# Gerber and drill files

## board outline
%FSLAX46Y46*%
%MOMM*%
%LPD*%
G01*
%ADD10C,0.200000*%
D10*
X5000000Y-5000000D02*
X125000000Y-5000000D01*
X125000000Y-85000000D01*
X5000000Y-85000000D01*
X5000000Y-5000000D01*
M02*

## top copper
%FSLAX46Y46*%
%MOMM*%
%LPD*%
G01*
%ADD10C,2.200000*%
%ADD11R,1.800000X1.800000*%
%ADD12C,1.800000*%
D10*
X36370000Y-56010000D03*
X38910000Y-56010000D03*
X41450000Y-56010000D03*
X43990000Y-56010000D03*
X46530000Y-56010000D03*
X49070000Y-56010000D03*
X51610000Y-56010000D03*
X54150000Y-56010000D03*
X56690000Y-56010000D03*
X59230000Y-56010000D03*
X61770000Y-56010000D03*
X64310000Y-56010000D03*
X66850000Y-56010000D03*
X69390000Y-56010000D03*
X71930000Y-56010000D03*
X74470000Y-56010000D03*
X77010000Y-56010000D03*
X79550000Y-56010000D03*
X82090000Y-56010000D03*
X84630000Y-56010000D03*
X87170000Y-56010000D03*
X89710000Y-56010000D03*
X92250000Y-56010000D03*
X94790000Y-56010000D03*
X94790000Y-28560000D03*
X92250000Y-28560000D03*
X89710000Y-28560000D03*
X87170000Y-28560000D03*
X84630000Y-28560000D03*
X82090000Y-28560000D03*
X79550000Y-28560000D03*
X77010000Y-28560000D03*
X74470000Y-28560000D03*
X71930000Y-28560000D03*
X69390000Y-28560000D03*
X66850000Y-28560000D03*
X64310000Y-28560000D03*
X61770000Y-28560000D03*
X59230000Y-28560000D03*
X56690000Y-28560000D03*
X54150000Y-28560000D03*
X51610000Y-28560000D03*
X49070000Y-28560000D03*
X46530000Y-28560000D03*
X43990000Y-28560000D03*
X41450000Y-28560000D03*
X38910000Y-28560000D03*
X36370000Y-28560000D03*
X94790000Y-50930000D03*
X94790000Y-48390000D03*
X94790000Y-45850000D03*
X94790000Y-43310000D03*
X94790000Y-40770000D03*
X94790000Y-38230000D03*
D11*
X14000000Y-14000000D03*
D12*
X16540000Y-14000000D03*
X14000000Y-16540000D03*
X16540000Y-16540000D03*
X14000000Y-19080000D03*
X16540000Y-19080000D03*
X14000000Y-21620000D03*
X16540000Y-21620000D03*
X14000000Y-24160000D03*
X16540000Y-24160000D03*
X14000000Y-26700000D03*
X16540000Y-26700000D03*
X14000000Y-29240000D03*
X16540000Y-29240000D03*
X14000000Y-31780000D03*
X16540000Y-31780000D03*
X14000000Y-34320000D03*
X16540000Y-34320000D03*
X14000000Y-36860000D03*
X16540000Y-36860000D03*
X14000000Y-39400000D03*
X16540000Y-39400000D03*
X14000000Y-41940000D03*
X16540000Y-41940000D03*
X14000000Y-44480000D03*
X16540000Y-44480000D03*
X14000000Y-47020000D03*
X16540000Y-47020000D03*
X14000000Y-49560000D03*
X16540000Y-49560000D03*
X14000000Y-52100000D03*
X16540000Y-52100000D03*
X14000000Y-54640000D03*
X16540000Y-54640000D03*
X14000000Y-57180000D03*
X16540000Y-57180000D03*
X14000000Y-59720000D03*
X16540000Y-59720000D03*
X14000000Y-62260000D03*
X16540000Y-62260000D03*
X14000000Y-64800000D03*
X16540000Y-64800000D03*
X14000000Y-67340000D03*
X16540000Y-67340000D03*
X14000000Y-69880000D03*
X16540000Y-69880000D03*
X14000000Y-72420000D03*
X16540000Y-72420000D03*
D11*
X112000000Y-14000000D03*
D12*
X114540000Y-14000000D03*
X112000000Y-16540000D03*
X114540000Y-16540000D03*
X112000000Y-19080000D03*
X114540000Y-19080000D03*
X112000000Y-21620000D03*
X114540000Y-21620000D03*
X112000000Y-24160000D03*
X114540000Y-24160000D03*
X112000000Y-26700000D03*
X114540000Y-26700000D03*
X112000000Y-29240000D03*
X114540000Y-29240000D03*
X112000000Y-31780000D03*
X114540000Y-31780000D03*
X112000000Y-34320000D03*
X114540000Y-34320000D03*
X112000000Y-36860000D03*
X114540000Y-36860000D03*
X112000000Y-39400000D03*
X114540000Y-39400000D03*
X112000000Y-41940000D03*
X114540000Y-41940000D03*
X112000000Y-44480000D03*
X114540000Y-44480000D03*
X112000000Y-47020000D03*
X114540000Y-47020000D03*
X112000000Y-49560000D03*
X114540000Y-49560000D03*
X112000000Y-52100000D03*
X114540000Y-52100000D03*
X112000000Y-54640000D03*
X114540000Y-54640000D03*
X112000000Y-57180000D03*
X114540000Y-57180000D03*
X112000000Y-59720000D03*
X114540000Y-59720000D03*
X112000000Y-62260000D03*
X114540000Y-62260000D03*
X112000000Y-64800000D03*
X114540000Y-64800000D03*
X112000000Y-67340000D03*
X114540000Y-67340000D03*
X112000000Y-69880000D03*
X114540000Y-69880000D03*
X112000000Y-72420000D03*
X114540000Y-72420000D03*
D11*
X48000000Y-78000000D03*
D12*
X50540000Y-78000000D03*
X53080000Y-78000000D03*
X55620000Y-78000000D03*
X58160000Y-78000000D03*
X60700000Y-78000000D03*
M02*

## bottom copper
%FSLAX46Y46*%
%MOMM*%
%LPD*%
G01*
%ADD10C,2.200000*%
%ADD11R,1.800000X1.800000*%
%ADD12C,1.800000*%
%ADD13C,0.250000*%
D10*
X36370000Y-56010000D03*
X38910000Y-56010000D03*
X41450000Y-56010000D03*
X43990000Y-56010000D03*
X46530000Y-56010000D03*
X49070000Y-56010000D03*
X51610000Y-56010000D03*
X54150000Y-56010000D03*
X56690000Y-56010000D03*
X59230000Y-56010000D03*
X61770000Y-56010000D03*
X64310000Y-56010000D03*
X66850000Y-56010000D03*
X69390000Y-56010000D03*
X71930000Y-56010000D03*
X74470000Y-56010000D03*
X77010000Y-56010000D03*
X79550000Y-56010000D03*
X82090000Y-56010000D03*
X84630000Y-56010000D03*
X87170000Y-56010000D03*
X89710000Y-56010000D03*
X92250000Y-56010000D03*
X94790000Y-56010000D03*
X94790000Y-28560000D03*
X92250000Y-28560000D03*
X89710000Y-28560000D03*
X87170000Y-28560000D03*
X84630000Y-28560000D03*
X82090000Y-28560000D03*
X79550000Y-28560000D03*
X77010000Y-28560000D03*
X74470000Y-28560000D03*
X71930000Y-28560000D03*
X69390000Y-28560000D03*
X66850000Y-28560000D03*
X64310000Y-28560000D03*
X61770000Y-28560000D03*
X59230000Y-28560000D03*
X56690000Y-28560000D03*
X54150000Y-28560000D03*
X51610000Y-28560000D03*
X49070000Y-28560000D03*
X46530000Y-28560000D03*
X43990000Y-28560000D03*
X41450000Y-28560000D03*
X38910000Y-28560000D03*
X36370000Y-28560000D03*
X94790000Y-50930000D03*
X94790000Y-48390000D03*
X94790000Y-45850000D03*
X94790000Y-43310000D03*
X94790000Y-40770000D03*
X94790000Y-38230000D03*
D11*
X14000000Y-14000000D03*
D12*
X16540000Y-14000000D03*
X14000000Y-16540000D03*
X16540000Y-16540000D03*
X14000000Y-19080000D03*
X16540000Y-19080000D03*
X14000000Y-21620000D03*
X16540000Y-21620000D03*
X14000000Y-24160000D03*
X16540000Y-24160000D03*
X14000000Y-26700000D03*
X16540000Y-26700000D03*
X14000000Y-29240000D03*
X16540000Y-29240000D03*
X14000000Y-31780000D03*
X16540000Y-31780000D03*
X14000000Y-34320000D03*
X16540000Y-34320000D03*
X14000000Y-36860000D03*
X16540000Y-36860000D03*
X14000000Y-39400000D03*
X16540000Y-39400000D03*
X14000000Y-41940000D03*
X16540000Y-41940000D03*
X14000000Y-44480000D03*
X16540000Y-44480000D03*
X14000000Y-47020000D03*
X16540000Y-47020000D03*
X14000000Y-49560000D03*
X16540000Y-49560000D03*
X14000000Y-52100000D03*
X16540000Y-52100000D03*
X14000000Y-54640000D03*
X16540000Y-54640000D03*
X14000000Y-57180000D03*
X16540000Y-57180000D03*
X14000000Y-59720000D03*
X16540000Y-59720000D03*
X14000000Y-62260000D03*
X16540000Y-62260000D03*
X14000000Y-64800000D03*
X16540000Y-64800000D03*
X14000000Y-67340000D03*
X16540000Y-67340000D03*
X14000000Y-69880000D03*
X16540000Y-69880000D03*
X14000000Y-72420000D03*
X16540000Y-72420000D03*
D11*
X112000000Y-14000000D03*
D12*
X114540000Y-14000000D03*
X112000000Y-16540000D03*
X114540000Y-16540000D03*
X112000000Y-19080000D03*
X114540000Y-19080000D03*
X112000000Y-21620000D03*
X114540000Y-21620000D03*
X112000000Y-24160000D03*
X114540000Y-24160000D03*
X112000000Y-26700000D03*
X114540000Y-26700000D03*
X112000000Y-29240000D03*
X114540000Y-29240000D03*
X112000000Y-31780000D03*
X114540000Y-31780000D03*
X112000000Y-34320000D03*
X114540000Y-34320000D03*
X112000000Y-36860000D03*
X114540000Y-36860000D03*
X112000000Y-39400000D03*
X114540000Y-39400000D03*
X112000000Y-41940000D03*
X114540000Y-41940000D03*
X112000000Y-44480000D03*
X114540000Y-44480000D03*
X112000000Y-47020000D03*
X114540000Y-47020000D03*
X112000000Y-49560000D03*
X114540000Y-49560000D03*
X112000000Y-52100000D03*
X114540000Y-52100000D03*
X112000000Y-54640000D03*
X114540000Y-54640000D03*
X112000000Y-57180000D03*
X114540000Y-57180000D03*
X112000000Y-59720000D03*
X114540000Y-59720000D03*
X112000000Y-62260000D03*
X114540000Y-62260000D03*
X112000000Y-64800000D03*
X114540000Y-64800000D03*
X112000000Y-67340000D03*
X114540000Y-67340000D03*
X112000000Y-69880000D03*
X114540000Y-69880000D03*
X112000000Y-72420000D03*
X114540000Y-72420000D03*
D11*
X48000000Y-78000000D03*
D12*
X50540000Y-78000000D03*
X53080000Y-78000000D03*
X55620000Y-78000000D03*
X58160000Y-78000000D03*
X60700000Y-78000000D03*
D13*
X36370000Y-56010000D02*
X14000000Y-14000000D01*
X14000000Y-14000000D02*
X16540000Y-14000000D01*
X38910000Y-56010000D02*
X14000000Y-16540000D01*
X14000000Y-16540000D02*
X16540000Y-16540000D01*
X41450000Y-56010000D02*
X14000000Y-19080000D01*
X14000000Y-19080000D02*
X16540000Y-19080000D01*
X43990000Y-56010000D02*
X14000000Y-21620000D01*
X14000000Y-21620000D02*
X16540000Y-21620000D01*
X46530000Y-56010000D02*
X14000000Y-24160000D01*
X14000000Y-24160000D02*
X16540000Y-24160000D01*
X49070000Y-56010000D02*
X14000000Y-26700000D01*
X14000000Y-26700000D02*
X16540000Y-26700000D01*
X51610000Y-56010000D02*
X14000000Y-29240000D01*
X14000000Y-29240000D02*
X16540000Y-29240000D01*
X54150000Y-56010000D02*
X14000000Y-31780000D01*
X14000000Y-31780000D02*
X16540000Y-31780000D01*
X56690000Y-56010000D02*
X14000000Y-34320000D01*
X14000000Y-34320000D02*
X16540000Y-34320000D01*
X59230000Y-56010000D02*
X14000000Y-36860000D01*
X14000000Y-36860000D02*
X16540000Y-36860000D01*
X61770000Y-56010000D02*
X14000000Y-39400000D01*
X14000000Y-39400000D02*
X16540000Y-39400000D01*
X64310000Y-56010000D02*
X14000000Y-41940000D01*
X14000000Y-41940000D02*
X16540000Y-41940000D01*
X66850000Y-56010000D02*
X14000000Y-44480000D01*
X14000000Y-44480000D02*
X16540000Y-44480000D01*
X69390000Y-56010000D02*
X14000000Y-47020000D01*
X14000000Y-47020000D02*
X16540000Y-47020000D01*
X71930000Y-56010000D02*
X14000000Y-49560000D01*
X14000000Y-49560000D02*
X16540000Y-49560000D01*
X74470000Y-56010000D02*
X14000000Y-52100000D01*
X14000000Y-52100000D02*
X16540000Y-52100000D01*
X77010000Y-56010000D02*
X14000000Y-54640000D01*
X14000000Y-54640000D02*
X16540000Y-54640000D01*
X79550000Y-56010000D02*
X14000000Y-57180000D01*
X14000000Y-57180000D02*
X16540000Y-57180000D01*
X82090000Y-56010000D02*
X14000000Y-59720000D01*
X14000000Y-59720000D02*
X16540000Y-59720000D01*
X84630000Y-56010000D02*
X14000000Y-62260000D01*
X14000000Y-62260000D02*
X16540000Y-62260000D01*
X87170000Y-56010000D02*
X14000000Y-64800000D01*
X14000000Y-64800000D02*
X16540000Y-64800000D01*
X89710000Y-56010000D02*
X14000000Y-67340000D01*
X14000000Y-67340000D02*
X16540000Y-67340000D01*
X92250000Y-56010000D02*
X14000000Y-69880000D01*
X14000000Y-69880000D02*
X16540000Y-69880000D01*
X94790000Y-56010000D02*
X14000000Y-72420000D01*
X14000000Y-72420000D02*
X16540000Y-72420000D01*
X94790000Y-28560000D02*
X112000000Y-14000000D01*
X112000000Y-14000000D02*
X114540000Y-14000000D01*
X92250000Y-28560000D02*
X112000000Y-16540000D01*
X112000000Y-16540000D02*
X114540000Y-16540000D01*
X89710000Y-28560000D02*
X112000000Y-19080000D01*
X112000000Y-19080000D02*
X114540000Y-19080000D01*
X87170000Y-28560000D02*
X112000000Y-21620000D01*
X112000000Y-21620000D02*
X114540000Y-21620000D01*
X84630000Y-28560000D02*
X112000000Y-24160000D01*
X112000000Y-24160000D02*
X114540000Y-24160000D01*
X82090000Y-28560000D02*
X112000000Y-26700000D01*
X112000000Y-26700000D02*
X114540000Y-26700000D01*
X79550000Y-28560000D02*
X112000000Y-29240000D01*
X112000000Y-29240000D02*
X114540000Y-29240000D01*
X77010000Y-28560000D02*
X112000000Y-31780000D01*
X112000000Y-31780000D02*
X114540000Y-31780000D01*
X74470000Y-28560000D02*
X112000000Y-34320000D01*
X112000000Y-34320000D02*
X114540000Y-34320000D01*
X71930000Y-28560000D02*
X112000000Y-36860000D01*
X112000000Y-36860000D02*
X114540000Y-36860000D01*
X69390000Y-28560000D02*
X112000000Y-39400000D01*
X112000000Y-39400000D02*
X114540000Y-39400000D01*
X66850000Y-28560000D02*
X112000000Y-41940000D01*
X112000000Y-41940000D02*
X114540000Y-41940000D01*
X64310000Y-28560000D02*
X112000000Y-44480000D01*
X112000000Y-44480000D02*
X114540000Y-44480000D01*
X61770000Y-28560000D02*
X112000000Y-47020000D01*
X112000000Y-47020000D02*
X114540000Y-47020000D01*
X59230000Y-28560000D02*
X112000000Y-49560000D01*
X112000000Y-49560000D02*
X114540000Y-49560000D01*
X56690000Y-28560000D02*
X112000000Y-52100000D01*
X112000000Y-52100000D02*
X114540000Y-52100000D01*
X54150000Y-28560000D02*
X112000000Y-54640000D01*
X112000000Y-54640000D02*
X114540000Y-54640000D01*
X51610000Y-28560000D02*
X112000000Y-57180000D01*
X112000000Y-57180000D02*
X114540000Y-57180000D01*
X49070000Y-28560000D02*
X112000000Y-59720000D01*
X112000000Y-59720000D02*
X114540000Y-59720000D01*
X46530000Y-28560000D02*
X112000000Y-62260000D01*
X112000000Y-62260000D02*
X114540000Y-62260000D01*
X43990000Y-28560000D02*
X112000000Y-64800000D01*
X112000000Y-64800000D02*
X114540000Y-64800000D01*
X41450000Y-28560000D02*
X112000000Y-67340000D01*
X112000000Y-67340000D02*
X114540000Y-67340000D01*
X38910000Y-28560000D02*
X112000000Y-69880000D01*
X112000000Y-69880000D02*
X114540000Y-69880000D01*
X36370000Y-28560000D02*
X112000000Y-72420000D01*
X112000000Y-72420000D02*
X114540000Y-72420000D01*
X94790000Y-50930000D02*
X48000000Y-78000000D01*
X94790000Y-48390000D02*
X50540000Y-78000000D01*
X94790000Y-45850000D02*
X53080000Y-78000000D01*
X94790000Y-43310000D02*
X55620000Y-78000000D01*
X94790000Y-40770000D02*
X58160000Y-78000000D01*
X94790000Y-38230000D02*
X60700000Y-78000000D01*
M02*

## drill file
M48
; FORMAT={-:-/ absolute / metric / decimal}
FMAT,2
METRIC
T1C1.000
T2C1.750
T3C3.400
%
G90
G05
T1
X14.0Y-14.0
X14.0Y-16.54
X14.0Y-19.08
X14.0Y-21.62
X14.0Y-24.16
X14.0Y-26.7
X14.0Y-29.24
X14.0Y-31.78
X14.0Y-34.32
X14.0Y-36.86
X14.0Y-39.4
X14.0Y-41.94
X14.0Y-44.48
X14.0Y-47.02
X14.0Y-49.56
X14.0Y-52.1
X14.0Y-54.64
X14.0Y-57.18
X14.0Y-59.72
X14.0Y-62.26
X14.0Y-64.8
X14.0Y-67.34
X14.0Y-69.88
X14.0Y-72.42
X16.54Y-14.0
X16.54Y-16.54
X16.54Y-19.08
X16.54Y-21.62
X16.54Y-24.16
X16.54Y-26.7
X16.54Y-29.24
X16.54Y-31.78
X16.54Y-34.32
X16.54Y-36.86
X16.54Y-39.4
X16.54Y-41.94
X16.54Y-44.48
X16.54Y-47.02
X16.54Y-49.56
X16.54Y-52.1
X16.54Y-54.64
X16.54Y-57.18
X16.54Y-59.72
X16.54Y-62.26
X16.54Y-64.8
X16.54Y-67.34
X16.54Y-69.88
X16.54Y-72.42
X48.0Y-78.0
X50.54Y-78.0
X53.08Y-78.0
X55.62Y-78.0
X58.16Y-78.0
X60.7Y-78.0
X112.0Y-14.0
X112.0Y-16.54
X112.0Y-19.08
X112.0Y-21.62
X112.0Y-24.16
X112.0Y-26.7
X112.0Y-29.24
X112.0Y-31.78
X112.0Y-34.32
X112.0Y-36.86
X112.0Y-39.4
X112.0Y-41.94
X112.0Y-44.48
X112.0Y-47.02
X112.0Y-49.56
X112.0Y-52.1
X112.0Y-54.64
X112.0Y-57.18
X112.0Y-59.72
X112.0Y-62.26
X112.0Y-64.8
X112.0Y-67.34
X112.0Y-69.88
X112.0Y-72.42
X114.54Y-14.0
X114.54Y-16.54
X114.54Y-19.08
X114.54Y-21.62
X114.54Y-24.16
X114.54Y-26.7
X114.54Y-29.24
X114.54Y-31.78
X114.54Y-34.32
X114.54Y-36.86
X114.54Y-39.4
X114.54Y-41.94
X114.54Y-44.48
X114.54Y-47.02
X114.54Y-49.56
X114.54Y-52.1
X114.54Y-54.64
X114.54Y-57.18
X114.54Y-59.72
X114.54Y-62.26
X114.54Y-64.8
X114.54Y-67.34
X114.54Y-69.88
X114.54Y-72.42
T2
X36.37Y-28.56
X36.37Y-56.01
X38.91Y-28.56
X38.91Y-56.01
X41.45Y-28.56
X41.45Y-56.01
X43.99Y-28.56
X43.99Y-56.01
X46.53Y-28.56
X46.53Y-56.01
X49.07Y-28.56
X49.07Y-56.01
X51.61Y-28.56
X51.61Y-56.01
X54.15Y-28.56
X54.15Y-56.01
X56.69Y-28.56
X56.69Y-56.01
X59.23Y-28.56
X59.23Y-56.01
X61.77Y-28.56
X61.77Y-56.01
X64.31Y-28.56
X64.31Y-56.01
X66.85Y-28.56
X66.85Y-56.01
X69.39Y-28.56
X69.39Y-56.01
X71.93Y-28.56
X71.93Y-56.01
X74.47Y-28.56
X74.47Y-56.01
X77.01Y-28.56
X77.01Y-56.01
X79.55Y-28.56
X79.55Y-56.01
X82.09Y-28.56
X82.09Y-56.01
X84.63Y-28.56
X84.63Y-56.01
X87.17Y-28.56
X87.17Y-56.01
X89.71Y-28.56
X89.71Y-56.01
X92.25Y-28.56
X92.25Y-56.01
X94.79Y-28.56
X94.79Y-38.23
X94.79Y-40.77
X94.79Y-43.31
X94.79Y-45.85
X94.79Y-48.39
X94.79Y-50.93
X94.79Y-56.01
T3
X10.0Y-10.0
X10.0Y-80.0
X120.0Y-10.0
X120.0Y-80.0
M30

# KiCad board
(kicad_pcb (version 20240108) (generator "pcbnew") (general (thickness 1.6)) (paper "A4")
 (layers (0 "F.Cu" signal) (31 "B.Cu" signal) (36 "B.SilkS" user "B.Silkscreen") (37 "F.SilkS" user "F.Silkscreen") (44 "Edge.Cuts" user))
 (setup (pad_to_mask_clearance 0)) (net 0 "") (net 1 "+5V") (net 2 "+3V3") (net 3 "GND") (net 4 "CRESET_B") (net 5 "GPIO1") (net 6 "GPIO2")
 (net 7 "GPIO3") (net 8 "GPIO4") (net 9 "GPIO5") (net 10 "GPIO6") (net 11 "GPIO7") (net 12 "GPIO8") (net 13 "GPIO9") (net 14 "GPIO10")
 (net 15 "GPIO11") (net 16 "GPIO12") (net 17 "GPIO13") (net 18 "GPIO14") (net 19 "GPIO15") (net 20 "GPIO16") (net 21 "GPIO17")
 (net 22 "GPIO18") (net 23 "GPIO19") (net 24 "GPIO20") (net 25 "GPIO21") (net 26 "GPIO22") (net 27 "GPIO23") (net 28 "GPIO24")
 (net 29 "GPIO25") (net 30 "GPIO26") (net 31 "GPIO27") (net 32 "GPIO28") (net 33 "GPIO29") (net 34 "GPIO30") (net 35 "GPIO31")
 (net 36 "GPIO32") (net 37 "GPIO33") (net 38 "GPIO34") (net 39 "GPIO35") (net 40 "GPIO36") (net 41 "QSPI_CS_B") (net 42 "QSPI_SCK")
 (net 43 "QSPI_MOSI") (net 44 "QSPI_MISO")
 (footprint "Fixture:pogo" (layer "F.Cu") (at 36.37 56.01)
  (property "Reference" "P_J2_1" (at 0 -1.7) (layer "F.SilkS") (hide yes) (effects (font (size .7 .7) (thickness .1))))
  (pad "1" thru_hole circle (at 0 0) (size 2.2 2.2) (drill 1.75) (layers "*.Cu" "*.Mask") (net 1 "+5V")))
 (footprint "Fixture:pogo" (layer "F.Cu") (at 38.91 56.01)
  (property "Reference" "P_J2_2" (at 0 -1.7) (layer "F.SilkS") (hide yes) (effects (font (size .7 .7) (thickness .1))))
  (pad "1" thru_hole circle (at 0 0) (size 2.2 2.2) (drill 1.75) (layers "*.Cu" "*.Mask") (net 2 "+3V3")))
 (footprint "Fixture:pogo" (layer "F.Cu") (at 41.449999999999996 56.01)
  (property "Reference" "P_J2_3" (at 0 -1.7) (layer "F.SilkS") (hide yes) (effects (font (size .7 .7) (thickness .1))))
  (pad "1" thru_hole circle (at 0 0) (size 2.2 2.2) (drill 1.75) (layers "*.Cu" "*.Mask") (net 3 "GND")))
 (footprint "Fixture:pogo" (layer "F.Cu") (at 43.989999999999995 56.01)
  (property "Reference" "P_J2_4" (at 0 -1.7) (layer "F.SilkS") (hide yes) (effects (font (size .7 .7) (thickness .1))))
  (pad "1" thru_hole circle (at 0 0) (size 2.2 2.2) (drill 1.75) (layers "*.Cu" "*.Mask") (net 3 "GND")))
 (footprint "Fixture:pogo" (layer "F.Cu") (at 46.53 56.01)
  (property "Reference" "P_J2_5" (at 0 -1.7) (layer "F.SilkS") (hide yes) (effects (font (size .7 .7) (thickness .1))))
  (pad "1" thru_hole circle (at 0 0) (size 2.2 2.2) (drill 1.75) (layers "*.Cu" "*.Mask") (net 3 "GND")))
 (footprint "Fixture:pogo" (layer "F.Cu") (at 49.06999999999999 56.01)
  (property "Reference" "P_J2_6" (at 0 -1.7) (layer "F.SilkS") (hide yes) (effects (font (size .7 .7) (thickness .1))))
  (pad "1" thru_hole circle (at 0 0) (size 2.2 2.2) (drill 1.75) (layers "*.Cu" "*.Mask") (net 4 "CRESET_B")))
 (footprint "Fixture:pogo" (layer "F.Cu") (at 51.61 56.01)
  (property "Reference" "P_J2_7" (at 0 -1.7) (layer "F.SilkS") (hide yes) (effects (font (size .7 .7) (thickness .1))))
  (pad "1" thru_hole circle (at 0 0) (size 2.2 2.2) (drill 1.75) (layers "*.Cu" "*.Mask") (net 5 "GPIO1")))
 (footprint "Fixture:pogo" (layer "F.Cu") (at 54.15 56.01)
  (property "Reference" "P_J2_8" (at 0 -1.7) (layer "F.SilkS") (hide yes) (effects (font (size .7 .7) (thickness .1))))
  (pad "1" thru_hole circle (at 0 0) (size 2.2 2.2) (drill 1.75) (layers "*.Cu" "*.Mask") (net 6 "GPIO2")))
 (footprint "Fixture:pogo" (layer "F.Cu") (at 56.69 56.01)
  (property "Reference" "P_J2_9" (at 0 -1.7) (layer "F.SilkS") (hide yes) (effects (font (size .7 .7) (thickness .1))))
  (pad "1" thru_hole circle (at 0 0) (size 2.2 2.2) (drill 1.75) (layers "*.Cu" "*.Mask") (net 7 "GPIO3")))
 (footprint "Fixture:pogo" (layer "F.Cu") (at 59.23 56.01)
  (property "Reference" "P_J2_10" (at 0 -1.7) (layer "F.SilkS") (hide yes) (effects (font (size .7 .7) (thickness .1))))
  (pad "1" thru_hole circle (at 0 0) (size 2.2 2.2) (drill 1.75) (layers "*.Cu" "*.Mask") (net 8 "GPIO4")))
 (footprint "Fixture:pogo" (layer "F.Cu") (at 61.769999999999996 56.01)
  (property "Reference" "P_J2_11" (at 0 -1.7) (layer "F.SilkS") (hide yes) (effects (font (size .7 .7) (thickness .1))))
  (pad "1" thru_hole circle (at 0 0) (size 2.2 2.2) (drill 1.75) (layers "*.Cu" "*.Mask") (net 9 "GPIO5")))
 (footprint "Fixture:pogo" (layer "F.Cu") (at 64.31 56.01)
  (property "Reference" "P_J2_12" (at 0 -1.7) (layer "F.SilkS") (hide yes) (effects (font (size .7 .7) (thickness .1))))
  (pad "1" thru_hole circle (at 0 0) (size 2.2 2.2) (drill 1.75) (layers "*.Cu" "*.Mask") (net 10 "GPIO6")))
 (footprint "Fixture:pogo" (layer "F.Cu") (at 66.85 56.01)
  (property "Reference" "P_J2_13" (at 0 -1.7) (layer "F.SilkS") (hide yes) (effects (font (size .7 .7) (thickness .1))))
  (pad "1" thru_hole circle (at 0 0) (size 2.2 2.2) (drill 1.75) (layers "*.Cu" "*.Mask") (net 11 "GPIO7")))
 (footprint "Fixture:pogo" (layer "F.Cu") (at 69.39 56.01)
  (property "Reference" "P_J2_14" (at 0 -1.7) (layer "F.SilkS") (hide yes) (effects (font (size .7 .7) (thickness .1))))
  (pad "1" thru_hole circle (at 0 0) (size 2.2 2.2) (drill 1.75) (layers "*.Cu" "*.Mask") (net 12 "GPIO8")))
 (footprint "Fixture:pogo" (layer "F.Cu") (at 71.93 56.01)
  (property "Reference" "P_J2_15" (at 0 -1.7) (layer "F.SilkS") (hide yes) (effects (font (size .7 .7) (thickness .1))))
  (pad "1" thru_hole circle (at 0 0) (size 2.2 2.2) (drill 1.75) (layers "*.Cu" "*.Mask") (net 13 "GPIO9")))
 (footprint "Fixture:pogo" (layer "F.Cu") (at 74.47 56.01)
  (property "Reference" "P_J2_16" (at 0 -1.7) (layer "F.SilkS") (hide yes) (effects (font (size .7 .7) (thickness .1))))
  (pad "1" thru_hole circle (at 0 0) (size 2.2 2.2) (drill 1.75) (layers "*.Cu" "*.Mask") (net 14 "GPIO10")))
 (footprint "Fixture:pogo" (layer "F.Cu") (at 77.00999999999999 56.01)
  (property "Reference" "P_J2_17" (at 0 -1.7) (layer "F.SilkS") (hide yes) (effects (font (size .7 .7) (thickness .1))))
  (pad "1" thru_hole circle (at 0 0) (size 2.2 2.2) (drill 1.75) (layers "*.Cu" "*.Mask") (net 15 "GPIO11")))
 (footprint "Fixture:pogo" (layer "F.Cu") (at 79.55 56.01)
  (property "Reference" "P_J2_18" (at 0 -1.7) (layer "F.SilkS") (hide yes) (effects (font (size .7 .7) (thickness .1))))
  (pad "1" thru_hole circle (at 0 0) (size 2.2 2.2) (drill 1.75) (layers "*.Cu" "*.Mask") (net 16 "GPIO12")))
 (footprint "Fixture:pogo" (layer "F.Cu") (at 82.09 56.01)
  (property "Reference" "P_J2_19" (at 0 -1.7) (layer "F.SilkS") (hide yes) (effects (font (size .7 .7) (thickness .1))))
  (pad "1" thru_hole circle (at 0 0) (size 2.2 2.2) (drill 1.75) (layers "*.Cu" "*.Mask") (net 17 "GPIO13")))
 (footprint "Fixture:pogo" (layer "F.Cu") (at 84.63 56.01)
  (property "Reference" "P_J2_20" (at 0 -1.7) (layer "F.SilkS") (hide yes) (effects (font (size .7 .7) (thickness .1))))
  (pad "1" thru_hole circle (at 0 0) (size 2.2 2.2) (drill 1.75) (layers "*.Cu" "*.Mask") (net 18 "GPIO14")))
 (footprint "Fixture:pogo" (layer "F.Cu") (at 87.16999999999999 56.01)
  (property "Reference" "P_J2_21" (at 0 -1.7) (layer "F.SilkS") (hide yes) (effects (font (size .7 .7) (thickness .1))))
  (pad "1" thru_hole circle (at 0 0) (size 2.2 2.2) (drill 1.75) (layers "*.Cu" "*.Mask") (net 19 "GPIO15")))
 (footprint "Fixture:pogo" (layer "F.Cu") (at 89.71000000000001 56.01)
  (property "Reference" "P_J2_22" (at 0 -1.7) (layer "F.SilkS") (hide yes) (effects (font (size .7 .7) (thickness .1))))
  (pad "1" thru_hole circle (at 0 0) (size 2.2 2.2) (drill 1.75) (layers "*.Cu" "*.Mask") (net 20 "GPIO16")))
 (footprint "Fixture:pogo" (layer "F.Cu") (at 92.25 56.01)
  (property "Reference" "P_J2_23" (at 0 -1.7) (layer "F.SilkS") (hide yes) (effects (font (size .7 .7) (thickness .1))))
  (pad "1" thru_hole circle (at 0 0) (size 2.2 2.2) (drill 1.75) (layers "*.Cu" "*.Mask") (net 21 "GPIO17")))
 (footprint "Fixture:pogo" (layer "F.Cu") (at 94.78999999999999 56.01)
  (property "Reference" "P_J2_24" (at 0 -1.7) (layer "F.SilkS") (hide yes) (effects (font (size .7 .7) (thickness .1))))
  (pad "1" thru_hole circle (at 0 0) (size 2.2 2.2) (drill 1.75) (layers "*.Cu" "*.Mask") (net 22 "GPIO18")))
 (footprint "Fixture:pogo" (layer "F.Cu") (at 94.79 28.56)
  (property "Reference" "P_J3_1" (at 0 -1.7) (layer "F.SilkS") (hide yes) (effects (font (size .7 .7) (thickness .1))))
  (pad "1" thru_hole circle (at 0 0) (size 2.2 2.2) (drill 1.75) (layers "*.Cu" "*.Mask") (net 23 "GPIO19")))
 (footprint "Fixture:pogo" (layer "F.Cu") (at 92.25 28.56)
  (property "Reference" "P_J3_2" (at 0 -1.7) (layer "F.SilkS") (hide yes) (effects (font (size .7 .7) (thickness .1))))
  (pad "1" thru_hole circle (at 0 0) (size 2.2 2.2) (drill 1.75) (layers "*.Cu" "*.Mask") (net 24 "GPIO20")))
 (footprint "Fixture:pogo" (layer "F.Cu") (at 89.71000000000001 28.56)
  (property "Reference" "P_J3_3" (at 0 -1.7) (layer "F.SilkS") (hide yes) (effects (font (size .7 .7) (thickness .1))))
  (pad "1" thru_hole circle (at 0 0) (size 2.2 2.2) (drill 1.75) (layers "*.Cu" "*.Mask") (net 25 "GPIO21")))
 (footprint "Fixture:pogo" (layer "F.Cu") (at 87.17 28.56)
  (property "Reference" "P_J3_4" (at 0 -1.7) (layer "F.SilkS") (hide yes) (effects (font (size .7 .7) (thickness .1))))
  (pad "1" thru_hole circle (at 0 0) (size 2.2 2.2) (drill 1.75) (layers "*.Cu" "*.Mask") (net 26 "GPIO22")))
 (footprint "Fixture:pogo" (layer "F.Cu") (at 84.63000000000001 28.56)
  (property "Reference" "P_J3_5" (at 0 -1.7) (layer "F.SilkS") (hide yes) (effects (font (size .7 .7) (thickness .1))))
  (pad "1" thru_hole circle (at 0 0) (size 2.2 2.2) (drill 1.75) (layers "*.Cu" "*.Mask") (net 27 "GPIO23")))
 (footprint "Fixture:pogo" (layer "F.Cu") (at 82.09 28.56)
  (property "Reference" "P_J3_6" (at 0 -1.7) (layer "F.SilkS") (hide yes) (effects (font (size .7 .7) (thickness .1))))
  (pad "1" thru_hole circle (at 0 0) (size 2.2 2.2) (drill 1.75) (layers "*.Cu" "*.Mask") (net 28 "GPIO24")))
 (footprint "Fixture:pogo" (layer "F.Cu") (at 79.55000000000001 28.56)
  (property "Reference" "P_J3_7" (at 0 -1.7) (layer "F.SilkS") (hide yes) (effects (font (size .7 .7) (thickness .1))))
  (pad "1" thru_hole circle (at 0 0) (size 2.2 2.2) (drill 1.75) (layers "*.Cu" "*.Mask") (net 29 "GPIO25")))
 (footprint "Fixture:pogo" (layer "F.Cu") (at 77.01 28.56)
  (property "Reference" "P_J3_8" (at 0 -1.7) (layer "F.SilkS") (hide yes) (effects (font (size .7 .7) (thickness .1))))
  (pad "1" thru_hole circle (at 0 0) (size 2.2 2.2) (drill 1.75) (layers "*.Cu" "*.Mask") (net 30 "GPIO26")))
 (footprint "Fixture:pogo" (layer "F.Cu") (at 74.47 28.56)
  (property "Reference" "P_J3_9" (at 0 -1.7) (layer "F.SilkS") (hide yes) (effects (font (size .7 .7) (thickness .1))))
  (pad "1" thru_hole circle (at 0 0) (size 2.2 2.2) (drill 1.75) (layers "*.Cu" "*.Mask") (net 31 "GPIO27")))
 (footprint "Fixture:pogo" (layer "F.Cu") (at 71.93 28.56)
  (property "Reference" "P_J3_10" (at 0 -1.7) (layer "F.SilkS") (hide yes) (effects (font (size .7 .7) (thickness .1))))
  (pad "1" thru_hole circle (at 0 0) (size 2.2 2.2) (drill 1.75) (layers "*.Cu" "*.Mask") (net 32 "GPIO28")))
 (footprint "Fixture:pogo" (layer "F.Cu") (at 69.39000000000001 28.56)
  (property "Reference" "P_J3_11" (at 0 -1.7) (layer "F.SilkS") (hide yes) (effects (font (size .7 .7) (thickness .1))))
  (pad "1" thru_hole circle (at 0 0) (size 2.2 2.2) (drill 1.75) (layers "*.Cu" "*.Mask") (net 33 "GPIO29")))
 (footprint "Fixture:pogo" (layer "F.Cu") (at 66.85000000000001 28.56)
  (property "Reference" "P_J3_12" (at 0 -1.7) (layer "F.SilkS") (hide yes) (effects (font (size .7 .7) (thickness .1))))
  (pad "1" thru_hole circle (at 0 0) (size 2.2 2.2) (drill 1.75) (layers "*.Cu" "*.Mask") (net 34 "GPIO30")))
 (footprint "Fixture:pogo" (layer "F.Cu") (at 64.31 28.56)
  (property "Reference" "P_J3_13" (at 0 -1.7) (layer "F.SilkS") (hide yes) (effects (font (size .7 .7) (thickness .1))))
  (pad "1" thru_hole circle (at 0 0) (size 2.2 2.2) (drill 1.75) (layers "*.Cu" "*.Mask") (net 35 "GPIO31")))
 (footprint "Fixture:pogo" (layer "F.Cu") (at 61.77 28.56)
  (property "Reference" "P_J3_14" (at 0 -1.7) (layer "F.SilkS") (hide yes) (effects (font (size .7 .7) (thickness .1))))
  (pad "1" thru_hole circle (at 0 0) (size 2.2 2.2) (drill 1.75) (layers "*.Cu" "*.Mask") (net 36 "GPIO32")))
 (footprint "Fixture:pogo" (layer "F.Cu") (at 59.230000000000004 28.56)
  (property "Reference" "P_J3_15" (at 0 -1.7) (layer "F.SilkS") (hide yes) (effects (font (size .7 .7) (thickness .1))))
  (pad "1" thru_hole circle (at 0 0) (size 2.2 2.2) (drill 1.75) (layers "*.Cu" "*.Mask") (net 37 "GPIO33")))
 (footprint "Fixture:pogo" (layer "F.Cu") (at 56.690000000000005 28.56)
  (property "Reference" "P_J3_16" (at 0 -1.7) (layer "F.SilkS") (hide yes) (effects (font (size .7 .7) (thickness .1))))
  (pad "1" thru_hole circle (at 0 0) (size 2.2 2.2) (drill 1.75) (layers "*.Cu" "*.Mask") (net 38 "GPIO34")))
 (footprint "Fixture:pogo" (layer "F.Cu") (at 54.150000000000006 28.56)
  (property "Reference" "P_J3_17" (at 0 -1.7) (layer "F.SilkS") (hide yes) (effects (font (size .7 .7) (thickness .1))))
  (pad "1" thru_hole circle (at 0 0) (size 2.2 2.2) (drill 1.75) (layers "*.Cu" "*.Mask") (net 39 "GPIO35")))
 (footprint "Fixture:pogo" (layer "F.Cu") (at 51.61000000000001 28.56)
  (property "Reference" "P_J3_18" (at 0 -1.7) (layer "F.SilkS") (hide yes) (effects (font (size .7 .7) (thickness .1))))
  (pad "1" thru_hole circle (at 0 0) (size 2.2 2.2) (drill 1.75) (layers "*.Cu" "*.Mask") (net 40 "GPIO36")))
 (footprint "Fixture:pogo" (layer "F.Cu") (at 49.07000000000001 28.56)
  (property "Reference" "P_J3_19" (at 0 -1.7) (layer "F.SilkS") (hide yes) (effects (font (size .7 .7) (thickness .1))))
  (pad "1" thru_hole circle (at 0 0) (size 2.2 2.2) (drill 1.75) (layers "*.Cu" "*.Mask") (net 3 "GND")))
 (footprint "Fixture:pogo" (layer "F.Cu") (at 46.53000000000001 28.56)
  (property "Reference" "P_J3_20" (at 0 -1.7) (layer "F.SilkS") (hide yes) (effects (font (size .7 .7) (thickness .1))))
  (pad "1" thru_hole circle (at 0 0) (size 2.2 2.2) (drill 1.75) (layers "*.Cu" "*.Mask") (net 3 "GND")))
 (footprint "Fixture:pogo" (layer "F.Cu") (at 43.99000000000001 28.56)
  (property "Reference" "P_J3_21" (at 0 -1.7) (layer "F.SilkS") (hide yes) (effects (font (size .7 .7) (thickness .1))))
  (pad "1" thru_hole circle (at 0 0) (size 2.2 2.2) (drill 1.75) (layers "*.Cu" "*.Mask") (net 3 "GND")))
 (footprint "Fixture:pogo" (layer "F.Cu") (at 41.45 28.56)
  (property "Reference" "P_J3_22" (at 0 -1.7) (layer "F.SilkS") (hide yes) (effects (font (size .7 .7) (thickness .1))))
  (pad "1" thru_hole circle (at 0 0) (size 2.2 2.2) (drill 1.75) (layers "*.Cu" "*.Mask") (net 3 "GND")))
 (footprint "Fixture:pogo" (layer "F.Cu") (at 38.910000000000004 28.56)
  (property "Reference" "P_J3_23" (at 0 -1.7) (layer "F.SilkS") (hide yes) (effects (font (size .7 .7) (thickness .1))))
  (pad "1" thru_hole circle (at 0 0) (size 2.2 2.2) (drill 1.75) (layers "*.Cu" "*.Mask") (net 2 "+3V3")))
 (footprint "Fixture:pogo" (layer "F.Cu") (at 36.370000000000005 28.56)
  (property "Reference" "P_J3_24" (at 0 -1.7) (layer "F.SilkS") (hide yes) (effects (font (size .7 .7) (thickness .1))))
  (pad "1" thru_hole circle (at 0 0) (size 2.2 2.2) (drill 1.75) (layers "*.Cu" "*.Mask") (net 1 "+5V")))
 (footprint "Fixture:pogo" (layer "F.Cu") (at 94.79 50.93)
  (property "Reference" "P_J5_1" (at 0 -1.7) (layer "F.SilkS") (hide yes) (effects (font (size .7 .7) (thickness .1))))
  (pad "1" thru_hole circle (at 0 0) (size 2.2 2.2) (drill 1.75) (layers "*.Cu" "*.Mask") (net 3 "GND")))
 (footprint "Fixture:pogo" (layer "F.Cu") (at 94.79 48.39)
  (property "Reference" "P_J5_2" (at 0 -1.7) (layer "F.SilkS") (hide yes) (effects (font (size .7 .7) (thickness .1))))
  (pad "1" thru_hole circle (at 0 0) (size 2.2 2.2) (drill 1.75) (layers "*.Cu" "*.Mask") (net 4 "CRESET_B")))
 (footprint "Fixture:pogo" (layer "F.Cu") (at 94.79 45.85)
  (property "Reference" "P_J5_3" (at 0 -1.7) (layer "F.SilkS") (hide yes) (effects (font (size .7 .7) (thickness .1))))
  (pad "1" thru_hole circle (at 0 0) (size 2.2 2.2) (drill 1.75) (layers "*.Cu" "*.Mask") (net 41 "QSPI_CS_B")))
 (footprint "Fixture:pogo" (layer "F.Cu") (at 94.79 43.31)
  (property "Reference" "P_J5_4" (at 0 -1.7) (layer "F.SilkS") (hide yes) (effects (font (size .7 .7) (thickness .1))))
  (pad "1" thru_hole circle (at 0 0) (size 2.2 2.2) (drill 1.75) (layers "*.Cu" "*.Mask") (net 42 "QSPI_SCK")))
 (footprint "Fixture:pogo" (layer "F.Cu") (at 94.79 40.769999999999996)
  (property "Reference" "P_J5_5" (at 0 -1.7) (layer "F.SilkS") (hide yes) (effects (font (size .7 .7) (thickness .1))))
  (pad "1" thru_hole circle (at 0 0) (size 2.2 2.2) (drill 1.75) (layers "*.Cu" "*.Mask") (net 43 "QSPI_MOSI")))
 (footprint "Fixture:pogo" (layer "F.Cu") (at 94.79 38.230000000000004)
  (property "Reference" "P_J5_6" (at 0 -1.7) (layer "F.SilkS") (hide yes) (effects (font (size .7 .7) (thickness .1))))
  (pad "1" thru_hole circle (at 0 0) (size 2.2 2.2) (drill 1.75) (layers "*.Cu" "*.Mask") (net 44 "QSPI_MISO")))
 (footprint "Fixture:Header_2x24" (layer "F.Cu") (at 14 14)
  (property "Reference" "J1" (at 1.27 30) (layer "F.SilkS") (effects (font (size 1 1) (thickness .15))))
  (pad "1" thru_hole rect (at 0 0) (size 1.8 1.8) (drill 1) (layers "*.Cu" "*.Mask") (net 1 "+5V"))
  (pad "1" thru_hole circle (at 2.54 0) (size 1.8 1.8) (drill 1) (layers "*.Cu" "*.Mask") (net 1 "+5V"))
  (pad "2" thru_hole circle (at 0 2.54) (size 1.8 1.8) (drill 1) (layers "*.Cu" "*.Mask") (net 2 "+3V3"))
  (pad "2" thru_hole circle (at 2.54 2.54) (size 1.8 1.8) (drill 1) (layers "*.Cu" "*.Mask") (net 2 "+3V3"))
  (pad "3" thru_hole circle (at 0 5.08) (size 1.8 1.8) (drill 1) (layers "*.Cu" "*.Mask") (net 3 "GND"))
  (pad "3" thru_hole circle (at 2.54 5.08) (size 1.8 1.8) (drill 1) (layers "*.Cu" "*.Mask") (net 3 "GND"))
  (pad "4" thru_hole circle (at 0 7.62) (size 1.8 1.8) (drill 1) (layers "*.Cu" "*.Mask") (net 3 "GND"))
  (pad "4" thru_hole circle (at 2.54 7.62) (size 1.8 1.8) (drill 1) (layers "*.Cu" "*.Mask") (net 3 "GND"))
  (pad "5" thru_hole circle (at 0 10.16) (size 1.8 1.8) (drill 1) (layers "*.Cu" "*.Mask") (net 3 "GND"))
  (pad "5" thru_hole circle (at 2.54 10.16) (size 1.8 1.8) (drill 1) (layers "*.Cu" "*.Mask") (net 3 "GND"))
  (pad "6" thru_hole circle (at 0 12.7) (size 1.8 1.8) (drill 1) (layers "*.Cu" "*.Mask") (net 4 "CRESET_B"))
  (pad "6" thru_hole circle (at 2.54 12.7) (size 1.8 1.8) (drill 1) (layers "*.Cu" "*.Mask") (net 4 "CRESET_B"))
  (pad "7" thru_hole circle (at 0 15.24) (size 1.8 1.8) (drill 1) (layers "*.Cu" "*.Mask") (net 5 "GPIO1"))
  (pad "7" thru_hole circle (at 2.54 15.24) (size 1.8 1.8) (drill 1) (layers "*.Cu" "*.Mask") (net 5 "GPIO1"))
  (pad "8" thru_hole circle (at 0 17.78) (size 1.8 1.8) (drill 1) (layers "*.Cu" "*.Mask") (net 6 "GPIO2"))
  (pad "8" thru_hole circle (at 2.54 17.78) (size 1.8 1.8) (drill 1) (layers "*.Cu" "*.Mask") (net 6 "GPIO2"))
  (pad "9" thru_hole circle (at 0 20.32) (size 1.8 1.8) (drill 1) (layers "*.Cu" "*.Mask") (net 7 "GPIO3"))
  (pad "9" thru_hole circle (at 2.54 20.32) (size 1.8 1.8) (drill 1) (layers "*.Cu" "*.Mask") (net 7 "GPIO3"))
  (pad "10" thru_hole circle (at 0 22.86) (size 1.8 1.8) (drill 1) (layers "*.Cu" "*.Mask") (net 8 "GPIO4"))
  (pad "10" thru_hole circle (at 2.54 22.86) (size 1.8 1.8) (drill 1) (layers "*.Cu" "*.Mask") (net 8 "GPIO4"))
  (pad "11" thru_hole circle (at 0 25.4) (size 1.8 1.8) (drill 1) (layers "*.Cu" "*.Mask") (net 9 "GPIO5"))
  (pad "11" thru_hole circle (at 2.54 25.4) (size 1.8 1.8) (drill 1) (layers "*.Cu" "*.Mask") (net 9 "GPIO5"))
  (pad "12" thru_hole circle (at 0 27.94) (size 1.8 1.8) (drill 1) (layers "*.Cu" "*.Mask") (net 10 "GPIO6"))
  (pad "12" thru_hole circle (at 2.54 27.94) (size 1.8 1.8) (drill 1) (layers "*.Cu" "*.Mask") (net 10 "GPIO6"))
  (pad "13" thru_hole circle (at 0 30.48) (size 1.8 1.8) (drill 1) (layers "*.Cu" "*.Mask") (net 11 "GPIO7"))
  (pad "13" thru_hole circle (at 2.54 30.48) (size 1.8 1.8) (drill 1) (layers "*.Cu" "*.Mask") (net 11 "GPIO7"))
  (pad "14" thru_hole circle (at 0 33.02) (size 1.8 1.8) (drill 1) (layers "*.Cu" "*.Mask") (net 12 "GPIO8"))
  (pad "14" thru_hole circle (at 2.54 33.02) (size 1.8 1.8) (drill 1) (layers "*.Cu" "*.Mask") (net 12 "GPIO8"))
  (pad "15" thru_hole circle (at 0 35.56) (size 1.8 1.8) (drill 1) (layers "*.Cu" "*.Mask") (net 13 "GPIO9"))
  (pad "15" thru_hole circle (at 2.54 35.56) (size 1.8 1.8) (drill 1) (layers "*.Cu" "*.Mask") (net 13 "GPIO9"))
  (pad "16" thru_hole circle (at 0 38.1) (size 1.8 1.8) (drill 1) (layers "*.Cu" "*.Mask") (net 14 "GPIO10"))
  (pad "16" thru_hole circle (at 2.54 38.1) (size 1.8 1.8) (drill 1) (layers "*.Cu" "*.Mask") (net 14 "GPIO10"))
  (pad "17" thru_hole circle (at 0 40.64) (size 1.8 1.8) (drill 1) (layers "*.Cu" "*.Mask") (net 15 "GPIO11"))
  (pad "17" thru_hole circle (at 2.54 40.64) (size 1.8 1.8) (drill 1) (layers "*.Cu" "*.Mask") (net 15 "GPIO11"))
  (pad "18" thru_hole circle (at 0 43.18) (size 1.8 1.8) (drill 1) (layers "*.Cu" "*.Mask") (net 16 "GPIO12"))
  (pad "18" thru_hole circle (at 2.54 43.18) (size 1.8 1.8) (drill 1) (layers "*.Cu" "*.Mask") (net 16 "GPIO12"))
  (pad "19" thru_hole circle (at 0 45.72) (size 1.8 1.8) (drill 1) (layers "*.Cu" "*.Mask") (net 17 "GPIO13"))
  (pad "19" thru_hole circle (at 2.54 45.72) (size 1.8 1.8) (drill 1) (layers "*.Cu" "*.Mask") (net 17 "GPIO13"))
  (pad "20" thru_hole circle (at 0 48.26) (size 1.8 1.8) (drill 1) (layers "*.Cu" "*.Mask") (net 18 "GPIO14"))
  (pad "20" thru_hole circle (at 2.54 48.26) (size 1.8 1.8) (drill 1) (layers "*.Cu" "*.Mask") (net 18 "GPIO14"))
  (pad "21" thru_hole circle (at 0 50.8) (size 1.8 1.8) (drill 1) (layers "*.Cu" "*.Mask") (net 19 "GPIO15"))
  (pad "21" thru_hole circle (at 2.54 50.8) (size 1.8 1.8) (drill 1) (layers "*.Cu" "*.Mask") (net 19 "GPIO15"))
  (pad "22" thru_hole circle (at 0 53.34) (size 1.8 1.8) (drill 1) (layers "*.Cu" "*.Mask") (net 20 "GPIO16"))
  (pad "22" thru_hole circle (at 2.54 53.34) (size 1.8 1.8) (drill 1) (layers "*.Cu" "*.Mask") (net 20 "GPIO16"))
  (pad "23" thru_hole circle (at 0 55.88) (size 1.8 1.8) (drill 1) (layers "*.Cu" "*.Mask") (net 21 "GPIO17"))
  (pad "23" thru_hole circle (at 2.54 55.88) (size 1.8 1.8) (drill 1) (layers "*.Cu" "*.Mask") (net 21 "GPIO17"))
  (pad "24" thru_hole circle (at 0 58.42) (size 1.8 1.8) (drill 1) (layers "*.Cu" "*.Mask") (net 22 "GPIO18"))
  (pad "24" thru_hole circle (at 2.54 58.42) (size 1.8 1.8) (drill 1) (layers "*.Cu" "*.Mask") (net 22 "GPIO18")))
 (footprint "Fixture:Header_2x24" (layer "F.Cu") (at 112 14)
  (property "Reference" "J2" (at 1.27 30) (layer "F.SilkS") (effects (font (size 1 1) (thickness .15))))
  (pad "1" thru_hole rect (at 0 0) (size 1.8 1.8) (drill 1) (layers "*.Cu" "*.Mask") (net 23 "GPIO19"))
  (pad "1" thru_hole circle (at 2.54 0) (size 1.8 1.8) (drill 1) (layers "*.Cu" "*.Mask") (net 23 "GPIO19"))
  (pad "2" thru_hole circle (at 0 2.54) (size 1.8 1.8) (drill 1) (layers "*.Cu" "*.Mask") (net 24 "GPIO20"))
  (pad "2" thru_hole circle (at 2.54 2.54) (size 1.8 1.8) (drill 1) (layers "*.Cu" "*.Mask") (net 24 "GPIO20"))
  (pad "3" thru_hole circle (at 0 5.08) (size 1.8 1.8) (drill 1) (layers "*.Cu" "*.Mask") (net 25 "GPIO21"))
  (pad "3" thru_hole circle (at 2.54 5.08) (size 1.8 1.8) (drill 1) (layers "*.Cu" "*.Mask") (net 25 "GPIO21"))
  (pad "4" thru_hole circle (at 0 7.62) (size 1.8 1.8) (drill 1) (layers "*.Cu" "*.Mask") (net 26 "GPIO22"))
  (pad "4" thru_hole circle (at 2.54 7.62) (size 1.8 1.8) (drill 1) (layers "*.Cu" "*.Mask") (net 26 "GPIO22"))
  (pad "5" thru_hole circle (at 0 10.16) (size 1.8 1.8) (drill 1) (layers "*.Cu" "*.Mask") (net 27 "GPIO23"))
  (pad "5" thru_hole circle (at 2.54 10.16) (size 1.8 1.8) (drill 1) (layers "*.Cu" "*.Mask") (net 27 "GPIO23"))
  (pad "6" thru_hole circle (at 0 12.7) (size 1.8 1.8) (drill 1) (layers "*.Cu" "*.Mask") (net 28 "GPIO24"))
  (pad "6" thru_hole circle (at 2.54 12.7) (size 1.8 1.8) (drill 1) (layers "*.Cu" "*.Mask") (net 28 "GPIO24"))
  (pad "7" thru_hole circle (at 0 15.24) (size 1.8 1.8) (drill 1) (layers "*.Cu" "*.Mask") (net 29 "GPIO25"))
  (pad "7" thru_hole circle (at 2.54 15.24) (size 1.8 1.8) (drill 1) (layers "*.Cu" "*.Mask") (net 29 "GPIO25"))
  (pad "8" thru_hole circle (at 0 17.78) (size 1.8 1.8) (drill 1) (layers "*.Cu" "*.Mask") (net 30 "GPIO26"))
  (pad "8" thru_hole circle (at 2.54 17.78) (size 1.8 1.8) (drill 1) (layers "*.Cu" "*.Mask") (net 30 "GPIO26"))
  (pad "9" thru_hole circle (at 0 20.32) (size 1.8 1.8) (drill 1) (layers "*.Cu" "*.Mask") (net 31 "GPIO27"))
  (pad "9" thru_hole circle (at 2.54 20.32) (size 1.8 1.8) (drill 1) (layers "*.Cu" "*.Mask") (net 31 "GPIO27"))
  (pad "10" thru_hole circle (at 0 22.86) (size 1.8 1.8) (drill 1) (layers "*.Cu" "*.Mask") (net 32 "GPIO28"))
  (pad "10" thru_hole circle (at 2.54 22.86) (size 1.8 1.8) (drill 1) (layers "*.Cu" "*.Mask") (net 32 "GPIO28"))
  (pad "11" thru_hole circle (at 0 25.4) (size 1.8 1.8) (drill 1) (layers "*.Cu" "*.Mask") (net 33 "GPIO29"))
  (pad "11" thru_hole circle (at 2.54 25.4) (size 1.8 1.8) (drill 1) (layers "*.Cu" "*.Mask") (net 33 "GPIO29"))
  (pad "12" thru_hole circle (at 0 27.94) (size 1.8 1.8) (drill 1) (layers "*.Cu" "*.Mask") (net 34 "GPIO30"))
  (pad "12" thru_hole circle (at 2.54 27.94) (size 1.8 1.8) (drill 1) (layers "*.Cu" "*.Mask") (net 34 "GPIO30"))
  (pad "13" thru_hole circle (at 0 30.48) (size 1.8 1.8) (drill 1) (layers "*.Cu" "*.Mask") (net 35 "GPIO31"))
  (pad "13" thru_hole circle (at 2.54 30.48) (size 1.8 1.8) (drill 1) (layers "*.Cu" "*.Mask") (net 35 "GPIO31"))
  (pad "14" thru_hole circle (at 0 33.02) (size 1.8 1.8) (drill 1) (layers "*.Cu" "*.Mask") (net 36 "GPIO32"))
  (pad "14" thru_hole circle (at 2.54 33.02) (size 1.8 1.8) (drill 1) (layers "*.Cu" "*.Mask") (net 36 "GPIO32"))
  (pad "15" thru_hole circle (at 0 35.56) (size 1.8 1.8) (drill 1) (layers "*.Cu" "*.Mask") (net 37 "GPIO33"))
  (pad "15" thru_hole circle (at 2.54 35.56) (size 1.8 1.8) (drill 1) (layers "*.Cu" "*.Mask") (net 37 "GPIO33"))
  (pad "16" thru_hole circle (at 0 38.1) (size 1.8 1.8) (drill 1) (layers "*.Cu" "*.Mask") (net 38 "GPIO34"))
  (pad "16" thru_hole circle (at 2.54 38.1) (size 1.8 1.8) (drill 1) (layers "*.Cu" "*.Mask") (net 38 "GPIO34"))
  (pad "17" thru_hole circle (at 0 40.64) (size 1.8 1.8) (drill 1) (layers "*.Cu" "*.Mask") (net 39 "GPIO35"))
  (pad "17" thru_hole circle (at 2.54 40.64) (size 1.8 1.8) (drill 1) (layers "*.Cu" "*.Mask") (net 39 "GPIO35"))
  (pad "18" thru_hole circle (at 0 43.18) (size 1.8 1.8) (drill 1) (layers "*.Cu" "*.Mask") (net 40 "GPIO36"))
  (pad "18" thru_hole circle (at 2.54 43.18) (size 1.8 1.8) (drill 1) (layers "*.Cu" "*.Mask") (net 40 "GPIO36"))
  (pad "19" thru_hole circle (at 0 45.72) (size 1.8 1.8) (drill 1) (layers "*.Cu" "*.Mask") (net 3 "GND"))
  (pad "19" thru_hole circle (at 2.54 45.72) (size 1.8 1.8) (drill 1) (layers "*.Cu" "*.Mask") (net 3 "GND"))
  (pad "20" thru_hole circle (at 0 48.26) (size 1.8 1.8) (drill 1) (layers "*.Cu" "*.Mask") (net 3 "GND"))
  (pad "20" thru_hole circle (at 2.54 48.26) (size 1.8 1.8) (drill 1) (layers "*.Cu" "*.Mask") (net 3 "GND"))
  (pad "21" thru_hole circle (at 0 50.8) (size 1.8 1.8) (drill 1) (layers "*.Cu" "*.Mask") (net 3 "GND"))
  (pad "21" thru_hole circle (at 2.54 50.8) (size 1.8 1.8) (drill 1) (layers "*.Cu" "*.Mask") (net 3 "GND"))
  (pad "22" thru_hole circle (at 0 53.34) (size 1.8 1.8) (drill 1) (layers "*.Cu" "*.Mask") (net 3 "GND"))
  (pad "22" thru_hole circle (at 2.54 53.34) (size 1.8 1.8) (drill 1) (layers "*.Cu" "*.Mask") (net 3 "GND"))
  (pad "23" thru_hole circle (at 0 55.88) (size 1.8 1.8) (drill 1) (layers "*.Cu" "*.Mask") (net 2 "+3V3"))
  (pad "23" thru_hole circle (at 2.54 55.88) (size 1.8 1.8) (drill 1) (layers "*.Cu" "*.Mask") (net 2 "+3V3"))
  (pad "24" thru_hole circle (at 0 58.42) (size 1.8 1.8) (drill 1) (layers "*.Cu" "*.Mask") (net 1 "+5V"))
  (pad "24" thru_hole circle (at 2.54 58.42) (size 1.8 1.8) (drill 1) (layers "*.Cu" "*.Mask") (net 1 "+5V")))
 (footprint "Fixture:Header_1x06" (layer "F.Cu") (at 48 78)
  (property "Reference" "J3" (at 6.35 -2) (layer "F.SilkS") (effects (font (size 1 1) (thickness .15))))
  (pad "1" thru_hole rect (at 0 0) (size 1.8 1.8) (drill 1) (layers "*.Cu" "*.Mask") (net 3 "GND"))
  (pad "2" thru_hole circle (at 2.54 0) (size 1.8 1.8) (drill 1) (layers "*.Cu" "*.Mask") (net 4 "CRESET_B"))
  (pad "3" thru_hole circle (at 5.08 0) (size 1.8 1.8) (drill 1) (layers "*.Cu" "*.Mask") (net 41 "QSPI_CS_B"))
  (pad "4" thru_hole circle (at 7.62 0) (size 1.8 1.8) (drill 1) (layers "*.Cu" "*.Mask") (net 42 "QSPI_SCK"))
  (pad "5" thru_hole circle (at 10.16 0) (size 1.8 1.8) (drill 1) (layers "*.Cu" "*.Mask") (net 43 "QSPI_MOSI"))
  (pad "6" thru_hole circle (at 12.7 0) (size 1.8 1.8) (drill 1) (layers "*.Cu" "*.Mask") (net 44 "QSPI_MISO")))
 (gr_rect (start 5 5) (end 125 85) (stroke (width .2) (type solid)) (fill none) (layer "Edge.Cuts"))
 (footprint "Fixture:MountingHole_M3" (layer "F.Cu") (at 10 10)
  (pad "" np_thru_hole circle (at 0 0) (size 3.4 3.4) (drill 3.4) (layers "*.Cu" "*.Mask")))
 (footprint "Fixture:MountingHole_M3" (layer "F.Cu") (at 120 10)
  (pad "" np_thru_hole circle (at 0 0) (size 3.4 3.4) (drill 3.4) (layers "*.Cu" "*.Mask")))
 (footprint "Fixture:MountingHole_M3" (layer "F.Cu") (at 10 80)
  (pad "" np_thru_hole circle (at 0 0) (size 3.4 3.4) (drill 3.4) (layers "*.Cu" "*.Mask")))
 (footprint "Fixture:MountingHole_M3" (layer "F.Cu") (at 120 80)
  (pad "" np_thru_hole circle (at 0 0) (size 3.4 3.4) (drill 3.4) (layers "*.Cu" "*.Mask")))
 (segment (start 36.37 56.01) (end 14 14) (width 0.25) (layer "B.Cu") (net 1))
 (segment (start 14 14) (end 16.54 14) (width 0.25) (layer "B.Cu") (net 1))
 (segment (start 38.91 56.01) (end 14 16.54) (width 0.25) (layer "B.Cu") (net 2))
 (segment (start 14 16.54) (end 16.54 16.54) (width 0.25) (layer "B.Cu") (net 2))
 (segment (start 41.449999999999996 56.01) (end 14 19.08) (width 0.25) (layer "B.Cu") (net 3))
 (segment (start 14 19.08) (end 16.54 19.08) (width 0.25) (layer "B.Cu") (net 3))
 (segment (start 43.989999999999995 56.01) (end 14 21.62) (width 0.25) (layer "B.Cu") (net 3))
 (segment (start 14 21.62) (end 16.54 21.62) (width 0.25) (layer "B.Cu") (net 3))
 (segment (start 46.53 56.01) (end 14 24.16) (width 0.25) (layer "B.Cu") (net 3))
 (segment (start 14 24.16) (end 16.54 24.16) (width 0.25) (layer "B.Cu") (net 3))
 (segment (start 49.06999999999999 56.01) (end 14 26.7) (width 0.25) (layer "B.Cu") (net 4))
 (segment (start 14 26.7) (end 16.54 26.7) (width 0.25) (layer "B.Cu") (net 4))
 (segment (start 51.61 56.01) (end 14 29.240000000000002) (width 0.25) (layer "B.Cu") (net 5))
 (segment (start 14 29.240000000000002) (end 16.54 29.240000000000002) (width 0.25) (layer "B.Cu") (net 5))
 (segment (start 54.15 56.01) (end 14 31.78) (width 0.25) (layer "B.Cu") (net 6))
 (segment (start 14 31.78) (end 16.54 31.78) (width 0.25) (layer "B.Cu") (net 6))
 (segment (start 56.69 56.01) (end 14 34.32) (width 0.25) (layer "B.Cu") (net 7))
 (segment (start 14 34.32) (end 16.54 34.32) (width 0.25) (layer "B.Cu") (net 7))
 (segment (start 59.23 56.01) (end 14 36.86) (width 0.25) (layer "B.Cu") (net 8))
 (segment (start 14 36.86) (end 16.54 36.86) (width 0.25) (layer "B.Cu") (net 8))
 (segment (start 61.769999999999996 56.01) (end 14 39.4) (width 0.25) (layer "B.Cu") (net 9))
 (segment (start 14 39.4) (end 16.54 39.4) (width 0.25) (layer "B.Cu") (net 9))
 (segment (start 64.31 56.01) (end 14 41.94) (width 0.25) (layer "B.Cu") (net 10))
 (segment (start 14 41.94) (end 16.54 41.94) (width 0.25) (layer "B.Cu") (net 10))
 (segment (start 66.85 56.01) (end 14 44.480000000000004) (width 0.25) (layer "B.Cu") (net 11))
 (segment (start 14 44.480000000000004) (end 16.54 44.480000000000004) (width 0.25) (layer "B.Cu") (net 11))
 (segment (start 69.39 56.01) (end 14 47.02) (width 0.25) (layer "B.Cu") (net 12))
 (segment (start 14 47.02) (end 16.54 47.02) (width 0.25) (layer "B.Cu") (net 12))
 (segment (start 71.93 56.01) (end 14 49.56) (width 0.25) (layer "B.Cu") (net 13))
 (segment (start 14 49.56) (end 16.54 49.56) (width 0.25) (layer "B.Cu") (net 13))
 (segment (start 74.47 56.01) (end 14 52.1) (width 0.25) (layer "B.Cu") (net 14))
 (segment (start 14 52.1) (end 16.54 52.1) (width 0.25) (layer "B.Cu") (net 14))
 (segment (start 77.00999999999999 56.01) (end 14 54.64) (width 0.25) (layer "B.Cu") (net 15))
 (segment (start 14 54.64) (end 16.54 54.64) (width 0.25) (layer "B.Cu") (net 15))
 (segment (start 79.55 56.01) (end 14 57.18) (width 0.25) (layer "B.Cu") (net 16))
 (segment (start 14 57.18) (end 16.54 57.18) (width 0.25) (layer "B.Cu") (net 16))
 (segment (start 82.09 56.01) (end 14 59.72) (width 0.25) (layer "B.Cu") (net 17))
 (segment (start 14 59.72) (end 16.54 59.72) (width 0.25) (layer "B.Cu") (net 17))
 (segment (start 84.63 56.01) (end 14 62.26) (width 0.25) (layer "B.Cu") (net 18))
 (segment (start 14 62.26) (end 16.54 62.26) (width 0.25) (layer "B.Cu") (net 18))
 (segment (start 87.16999999999999 56.01) (end 14 64.8) (width 0.25) (layer "B.Cu") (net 19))
 (segment (start 14 64.8) (end 16.54 64.8) (width 0.25) (layer "B.Cu") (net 19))
 (segment (start 89.71000000000001 56.01) (end 14 67.34) (width 0.25) (layer "B.Cu") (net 20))
 (segment (start 14 67.34) (end 16.54 67.34) (width 0.25) (layer "B.Cu") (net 20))
 (segment (start 92.25 56.01) (end 14 69.88) (width 0.25) (layer "B.Cu") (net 21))
 (segment (start 14 69.88) (end 16.54 69.88) (width 0.25) (layer "B.Cu") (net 21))
 (segment (start 94.78999999999999 56.01) (end 14 72.42) (width 0.25) (layer "B.Cu") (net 22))
 (segment (start 14 72.42) (end 16.54 72.42) (width 0.25) (layer "B.Cu") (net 22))
 (segment (start 94.79 28.56) (end 112 14) (width 0.25) (layer "B.Cu") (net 23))
 (segment (start 112 14) (end 114.54 14) (width 0.25) (layer "B.Cu") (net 23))
 (segment (start 92.25 28.56) (end 112 16.54) (width 0.25) (layer "B.Cu") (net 24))
 (segment (start 112 16.54) (end 114.54 16.54) (width 0.25) (layer "B.Cu") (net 24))
 (segment (start 89.71000000000001 28.56) (end 112 19.08) (width 0.25) (layer "B.Cu") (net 25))
 (segment (start 112 19.08) (end 114.54 19.08) (width 0.25) (layer "B.Cu") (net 25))
 (segment (start 87.17 28.56) (end 112 21.62) (width 0.25) (layer "B.Cu") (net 26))
 (segment (start 112 21.62) (end 114.54 21.62) (width 0.25) (layer "B.Cu") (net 26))
 (segment (start 84.63000000000001 28.56) (end 112 24.16) (width 0.25) (layer "B.Cu") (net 27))
 (segment (start 112 24.16) (end 114.54 24.16) (width 0.25) (layer "B.Cu") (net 27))
 (segment (start 82.09 28.56) (end 112 26.7) (width 0.25) (layer "B.Cu") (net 28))
 (segment (start 112 26.7) (end 114.54 26.7) (width 0.25) (layer "B.Cu") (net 28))
 (segment (start 79.55000000000001 28.56) (end 112 29.240000000000002) (width 0.25) (layer "B.Cu") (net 29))
 (segment (start 112 29.240000000000002) (end 114.54 29.240000000000002) (width 0.25) (layer "B.Cu") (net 29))
 (segment (start 77.01 28.56) (end 112 31.78) (width 0.25) (layer "B.Cu") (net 30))
 (segment (start 112 31.78) (end 114.54 31.78) (width 0.25) (layer "B.Cu") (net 30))
 (segment (start 74.47 28.56) (end 112 34.32) (width 0.25) (layer "B.Cu") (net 31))
 (segment (start 112 34.32) (end 114.54 34.32) (width 0.25) (layer "B.Cu") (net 31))
 (segment (start 71.93 28.56) (end 112 36.86) (width 0.25) (layer "B.Cu") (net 32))
 (segment (start 112 36.86) (end 114.54 36.86) (width 0.25) (layer "B.Cu") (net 32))
 (segment (start 69.39000000000001 28.56) (end 112 39.4) (width 0.25) (layer "B.Cu") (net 33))
 (segment (start 112 39.4) (end 114.54 39.4) (width 0.25) (layer "B.Cu") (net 33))
 (segment (start 66.85000000000001 28.56) (end 112 41.94) (width 0.25) (layer "B.Cu") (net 34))
 (segment (start 112 41.94) (end 114.54 41.94) (width 0.25) (layer "B.Cu") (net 34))
 (segment (start 64.31 28.56) (end 112 44.480000000000004) (width 0.25) (layer "B.Cu") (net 35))
 (segment (start 112 44.480000000000004) (end 114.54 44.480000000000004) (width 0.25) (layer "B.Cu") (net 35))
 (segment (start 61.77 28.56) (end 112 47.02) (width 0.25) (layer "B.Cu") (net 36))
 (segment (start 112 47.02) (end 114.54 47.02) (width 0.25) (layer "B.Cu") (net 36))
 (segment (start 59.230000000000004 28.56) (end 112 49.56) (width 0.25) (layer "B.Cu") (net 37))
 (segment (start 112 49.56) (end 114.54 49.56) (width 0.25) (layer "B.Cu") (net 37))
 (segment (start 56.690000000000005 28.56) (end 112 52.1) (width 0.25) (layer "B.Cu") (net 38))
 (segment (start 112 52.1) (end 114.54 52.1) (width 0.25) (layer "B.Cu") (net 38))
 (segment (start 54.150000000000006 28.56) (end 112 54.64) (width 0.25) (layer "B.Cu") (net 39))
 (segment (start 112 54.64) (end 114.54 54.64) (width 0.25) (layer "B.Cu") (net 39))
 (segment (start 51.61000000000001 28.56) (end 112 57.18) (width 0.25) (layer "B.Cu") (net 40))
 (segment (start 112 57.18) (end 114.54 57.18) (width 0.25) (layer "B.Cu") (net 40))
 (segment (start 49.07000000000001 28.56) (end 112 59.72) (width 0.25) (layer "B.Cu") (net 3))
 (segment (start 112 59.72) (end 114.54 59.72) (width 0.25) (layer "B.Cu") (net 3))
 (segment (start 46.53000000000001 28.56) (end 112 62.26) (width 0.25) (layer "B.Cu") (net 3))
 (segment (start 112 62.26) (end 114.54 62.26) (width 0.25) (layer "B.Cu") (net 3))
 (segment (start 43.99000000000001 28.56) (end 112 64.8) (width 0.25) (layer "B.Cu") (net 3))
 (segment (start 112 64.8) (end 114.54 64.8) (width 0.25) (layer "B.Cu") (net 3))
 (segment (start 41.45 28.56) (end 112 67.34) (width 0.25) (layer "B.Cu") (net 3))
 (segment (start 112 67.34) (end 114.54 67.34) (width 0.25) (layer "B.Cu") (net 3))
 (segment (start 38.910000000000004 28.56) (end 112 69.88) (width 0.25) (layer "B.Cu") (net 2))
 (segment (start 112 69.88) (end 114.54 69.88) (width 0.25) (layer "B.Cu") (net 2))
 (segment (start 36.370000000000005 28.56) (end 112 72.42) (width 0.25) (layer "B.Cu") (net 1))
 (segment (start 112 72.42) (end 114.54 72.42) (width 0.25) (layer "B.Cu") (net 1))
 (segment (start 94.79 50.93) (end 48 78) (width 0.25) (layer "B.Cu") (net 3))
 (segment (start 94.79 48.39) (end 50.54 78) (width 0.25) (layer "B.Cu") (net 4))
 (segment (start 94.79 45.85) (end 53.08 78) (width 0.25) (layer "B.Cu") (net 41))
 (segment (start 94.79 43.31) (end 55.62 78) (width 0.25) (layer "B.Cu") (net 42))
 (segment (start 94.79 40.769999999999996) (end 58.16 78) (width 0.25) (layer "B.Cu") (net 43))
 (segment (start 94.79 38.230000000000004) (end 60.7 78) (width 0.25) (layer "B.Cu") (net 44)))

